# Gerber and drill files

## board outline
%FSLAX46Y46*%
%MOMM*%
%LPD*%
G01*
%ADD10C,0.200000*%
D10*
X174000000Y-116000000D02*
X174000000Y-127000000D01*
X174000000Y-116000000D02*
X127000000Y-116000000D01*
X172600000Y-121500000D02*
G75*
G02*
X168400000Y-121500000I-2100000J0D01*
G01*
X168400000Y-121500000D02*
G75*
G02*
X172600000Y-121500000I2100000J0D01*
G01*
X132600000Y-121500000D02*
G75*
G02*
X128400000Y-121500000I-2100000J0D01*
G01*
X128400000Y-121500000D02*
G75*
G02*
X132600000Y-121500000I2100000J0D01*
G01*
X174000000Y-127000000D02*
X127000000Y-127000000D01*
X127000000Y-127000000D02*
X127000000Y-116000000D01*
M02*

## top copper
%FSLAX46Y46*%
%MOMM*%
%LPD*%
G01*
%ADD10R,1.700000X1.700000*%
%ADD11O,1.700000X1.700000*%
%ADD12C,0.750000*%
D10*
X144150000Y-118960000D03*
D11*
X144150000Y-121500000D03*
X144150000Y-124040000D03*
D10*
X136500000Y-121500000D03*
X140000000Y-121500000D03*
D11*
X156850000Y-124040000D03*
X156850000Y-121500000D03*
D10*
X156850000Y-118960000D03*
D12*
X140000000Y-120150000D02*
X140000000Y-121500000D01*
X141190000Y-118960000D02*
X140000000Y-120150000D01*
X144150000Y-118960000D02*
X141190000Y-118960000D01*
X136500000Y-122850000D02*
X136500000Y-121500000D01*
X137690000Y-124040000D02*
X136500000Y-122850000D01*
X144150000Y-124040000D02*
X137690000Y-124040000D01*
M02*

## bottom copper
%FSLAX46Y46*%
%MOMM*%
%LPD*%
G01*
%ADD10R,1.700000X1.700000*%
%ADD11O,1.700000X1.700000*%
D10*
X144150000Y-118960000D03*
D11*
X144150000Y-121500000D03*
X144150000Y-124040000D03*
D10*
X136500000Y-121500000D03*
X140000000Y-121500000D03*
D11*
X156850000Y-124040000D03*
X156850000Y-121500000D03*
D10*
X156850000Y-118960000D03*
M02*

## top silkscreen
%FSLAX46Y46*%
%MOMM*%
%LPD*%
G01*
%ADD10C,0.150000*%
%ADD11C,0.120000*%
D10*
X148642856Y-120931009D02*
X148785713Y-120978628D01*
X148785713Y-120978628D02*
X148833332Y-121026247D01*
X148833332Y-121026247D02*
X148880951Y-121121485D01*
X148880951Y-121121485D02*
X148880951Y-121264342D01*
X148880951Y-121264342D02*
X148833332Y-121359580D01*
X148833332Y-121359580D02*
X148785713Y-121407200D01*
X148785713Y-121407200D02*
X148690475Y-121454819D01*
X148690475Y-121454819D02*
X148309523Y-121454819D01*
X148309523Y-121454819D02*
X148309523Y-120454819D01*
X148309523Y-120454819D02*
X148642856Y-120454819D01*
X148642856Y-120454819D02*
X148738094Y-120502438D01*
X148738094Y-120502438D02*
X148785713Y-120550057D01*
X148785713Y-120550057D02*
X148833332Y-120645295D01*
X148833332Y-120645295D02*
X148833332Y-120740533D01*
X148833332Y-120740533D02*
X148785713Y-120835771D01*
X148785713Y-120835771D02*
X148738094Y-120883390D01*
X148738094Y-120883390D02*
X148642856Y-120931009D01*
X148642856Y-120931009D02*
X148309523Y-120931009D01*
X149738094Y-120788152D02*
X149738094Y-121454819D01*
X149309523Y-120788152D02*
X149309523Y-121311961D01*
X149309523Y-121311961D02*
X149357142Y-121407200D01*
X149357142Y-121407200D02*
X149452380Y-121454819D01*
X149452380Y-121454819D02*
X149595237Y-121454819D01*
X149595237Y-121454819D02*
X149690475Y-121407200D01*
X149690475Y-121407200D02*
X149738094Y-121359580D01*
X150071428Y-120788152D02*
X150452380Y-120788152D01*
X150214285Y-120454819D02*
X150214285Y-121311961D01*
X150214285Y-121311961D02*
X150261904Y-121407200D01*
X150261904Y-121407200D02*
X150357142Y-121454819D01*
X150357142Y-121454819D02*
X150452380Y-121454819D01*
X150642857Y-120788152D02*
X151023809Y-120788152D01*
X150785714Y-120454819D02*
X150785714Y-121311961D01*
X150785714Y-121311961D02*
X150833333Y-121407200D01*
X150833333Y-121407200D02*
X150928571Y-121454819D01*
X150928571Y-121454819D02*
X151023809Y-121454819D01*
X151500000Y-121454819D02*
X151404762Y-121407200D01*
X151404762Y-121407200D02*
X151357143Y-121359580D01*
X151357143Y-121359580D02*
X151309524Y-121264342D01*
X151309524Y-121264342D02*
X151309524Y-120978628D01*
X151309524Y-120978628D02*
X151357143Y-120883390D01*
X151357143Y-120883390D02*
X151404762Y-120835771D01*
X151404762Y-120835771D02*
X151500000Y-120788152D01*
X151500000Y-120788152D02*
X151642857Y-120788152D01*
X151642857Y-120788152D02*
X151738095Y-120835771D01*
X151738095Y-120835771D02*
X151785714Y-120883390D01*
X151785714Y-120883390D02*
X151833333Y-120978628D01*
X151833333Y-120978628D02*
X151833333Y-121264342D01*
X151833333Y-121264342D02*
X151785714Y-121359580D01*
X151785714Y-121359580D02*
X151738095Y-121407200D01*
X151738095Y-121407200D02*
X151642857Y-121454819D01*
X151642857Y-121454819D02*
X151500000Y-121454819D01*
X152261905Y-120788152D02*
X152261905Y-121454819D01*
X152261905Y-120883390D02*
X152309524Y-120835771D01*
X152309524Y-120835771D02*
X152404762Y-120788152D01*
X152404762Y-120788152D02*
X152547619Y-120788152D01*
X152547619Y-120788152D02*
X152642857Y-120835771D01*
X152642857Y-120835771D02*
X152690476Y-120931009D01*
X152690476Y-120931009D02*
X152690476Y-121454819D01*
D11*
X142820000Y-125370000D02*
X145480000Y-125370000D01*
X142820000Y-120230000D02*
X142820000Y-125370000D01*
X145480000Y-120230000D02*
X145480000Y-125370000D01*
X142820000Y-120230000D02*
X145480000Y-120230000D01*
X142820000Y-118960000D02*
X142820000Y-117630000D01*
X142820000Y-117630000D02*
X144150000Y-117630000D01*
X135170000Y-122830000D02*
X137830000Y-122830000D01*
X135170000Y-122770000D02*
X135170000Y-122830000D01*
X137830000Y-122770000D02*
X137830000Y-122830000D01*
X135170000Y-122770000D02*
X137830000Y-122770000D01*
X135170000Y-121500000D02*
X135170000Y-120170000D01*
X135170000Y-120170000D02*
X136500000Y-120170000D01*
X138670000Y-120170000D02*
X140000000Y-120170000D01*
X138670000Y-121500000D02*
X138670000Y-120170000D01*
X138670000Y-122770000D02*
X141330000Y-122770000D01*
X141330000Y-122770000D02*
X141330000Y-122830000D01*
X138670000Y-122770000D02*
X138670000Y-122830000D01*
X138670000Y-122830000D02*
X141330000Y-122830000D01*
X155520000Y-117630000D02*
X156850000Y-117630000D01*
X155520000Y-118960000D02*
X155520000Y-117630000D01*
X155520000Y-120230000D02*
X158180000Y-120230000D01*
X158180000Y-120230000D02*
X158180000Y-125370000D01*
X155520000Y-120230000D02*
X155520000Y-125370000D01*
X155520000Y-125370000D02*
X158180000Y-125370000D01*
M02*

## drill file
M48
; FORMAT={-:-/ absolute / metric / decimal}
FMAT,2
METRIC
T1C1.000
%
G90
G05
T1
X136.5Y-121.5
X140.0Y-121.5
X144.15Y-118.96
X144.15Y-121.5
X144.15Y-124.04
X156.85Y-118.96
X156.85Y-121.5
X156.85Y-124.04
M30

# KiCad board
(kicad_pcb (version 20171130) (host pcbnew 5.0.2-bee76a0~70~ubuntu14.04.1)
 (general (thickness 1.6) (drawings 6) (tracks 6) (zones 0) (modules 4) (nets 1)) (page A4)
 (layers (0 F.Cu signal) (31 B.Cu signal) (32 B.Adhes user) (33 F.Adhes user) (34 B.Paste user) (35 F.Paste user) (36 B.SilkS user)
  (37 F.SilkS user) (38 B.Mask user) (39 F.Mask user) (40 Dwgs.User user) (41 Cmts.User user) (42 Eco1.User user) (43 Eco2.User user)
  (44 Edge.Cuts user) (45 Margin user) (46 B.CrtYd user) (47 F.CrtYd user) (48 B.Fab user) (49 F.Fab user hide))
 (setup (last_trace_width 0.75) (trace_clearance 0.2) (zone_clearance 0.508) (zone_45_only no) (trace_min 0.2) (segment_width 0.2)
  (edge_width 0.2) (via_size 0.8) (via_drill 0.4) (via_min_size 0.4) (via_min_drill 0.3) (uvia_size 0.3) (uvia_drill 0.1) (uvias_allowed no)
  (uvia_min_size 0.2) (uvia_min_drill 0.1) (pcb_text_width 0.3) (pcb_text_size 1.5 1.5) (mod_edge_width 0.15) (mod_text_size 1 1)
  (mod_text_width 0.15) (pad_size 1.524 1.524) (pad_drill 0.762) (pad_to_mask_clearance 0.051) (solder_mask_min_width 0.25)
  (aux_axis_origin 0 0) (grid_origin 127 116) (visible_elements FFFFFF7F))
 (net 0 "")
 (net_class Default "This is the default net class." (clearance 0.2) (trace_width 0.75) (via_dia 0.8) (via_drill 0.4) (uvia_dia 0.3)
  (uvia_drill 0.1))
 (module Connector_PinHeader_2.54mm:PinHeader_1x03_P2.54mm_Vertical (layer F.Cu) (at 144.15 118.96)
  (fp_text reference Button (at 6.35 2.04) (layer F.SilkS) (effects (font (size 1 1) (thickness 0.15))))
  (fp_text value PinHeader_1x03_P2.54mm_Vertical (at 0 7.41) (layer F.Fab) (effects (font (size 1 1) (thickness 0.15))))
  (fp_line (start -1.33 6.41) (end 1.33 6.41) (layer F.SilkS) (width 0.12))
  (fp_line (start -1.33 1.27) (end -1.33 6.41) (layer F.SilkS) (width 0.12))
  (fp_line (start 1.33 1.27) (end 1.33 6.41) (layer F.SilkS) (width 0.12))
  (fp_line (start -1.33 1.27) (end 1.33 1.27) (layer F.SilkS) (width 0.12))
  (fp_line (start -1.33 0) (end -1.33 -1.33) (layer F.SilkS) (width 0.12))
  (fp_line (start -1.33 -1.33) (end 0 -1.33) (layer F.SilkS) (width 0.12))
  (pad 1 thru_hole rect (at 0 0) (size 1.7 1.7) (drill 1) (layers *.Cu *.Mask))
  (pad 2 thru_hole oval (at 0 2.54) (size 1.7 1.7) (drill 1) (layers *.Cu *.Mask))
  (pad 3 thru_hole oval (at 0 5.08) (size 1.7 1.7) (drill 1) (layers *.Cu *.Mask)))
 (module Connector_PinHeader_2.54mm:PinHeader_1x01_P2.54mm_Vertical (layer F.Cu) (at 136.5 121.5)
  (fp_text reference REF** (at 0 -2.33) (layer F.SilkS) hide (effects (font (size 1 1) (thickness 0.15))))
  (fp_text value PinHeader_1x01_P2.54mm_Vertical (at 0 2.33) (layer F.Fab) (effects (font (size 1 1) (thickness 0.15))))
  (fp_line (start -1.33 1.33) (end 1.33 1.33) (layer F.SilkS) (width 0.12))
  (fp_line (start -1.33 1.27) (end -1.33 1.33) (layer F.SilkS) (width 0.12))
  (fp_line (start 1.33 1.27) (end 1.33 1.33) (layer F.SilkS) (width 0.12))
  (fp_line (start -1.33 1.27) (end 1.33 1.27) (layer F.SilkS) (width 0.12))
  (fp_line (start -1.33 0) (end -1.33 -1.33) (layer F.SilkS) (width 0.12))
  (fp_line (start -1.33 -1.33) (end 0 -1.33) (layer F.SilkS) (width 0.12))
  (pad 1 thru_hole rect (at 0 0) (size 1.7 1.7) (drill 1) (layers *.Cu *.Mask)))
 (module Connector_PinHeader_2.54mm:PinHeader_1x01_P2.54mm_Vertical (layer F.Cu) (at 140 121.5)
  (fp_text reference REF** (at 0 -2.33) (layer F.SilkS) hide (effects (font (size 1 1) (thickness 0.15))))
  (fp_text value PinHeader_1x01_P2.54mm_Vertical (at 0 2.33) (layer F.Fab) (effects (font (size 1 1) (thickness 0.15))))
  (fp_line (start -1.33 -1.33) (end 0 -1.33) (layer F.SilkS) (width 0.12))
  (fp_line (start -1.33 0) (end -1.33 -1.33) (layer F.SilkS) (width 0.12))
  (fp_line (start -1.33 1.27) (end 1.33 1.27) (layer F.SilkS) (width 0.12))
  (fp_line (start 1.33 1.27) (end 1.33 1.33) (layer F.SilkS) (width 0.12))
  (fp_line (start -1.33 1.27) (end -1.33 1.33) (layer F.SilkS) (width 0.12))
  (fp_line (start -1.33 1.33) (end 1.33 1.33) (layer F.SilkS) (width 0.12))
  (pad 1 thru_hole rect (at 0 0) (size 1.7 1.7) (drill 1) (layers *.Cu *.Mask)))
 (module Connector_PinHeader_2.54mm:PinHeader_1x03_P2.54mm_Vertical (layer F.Cu) (at 156.85 118.96)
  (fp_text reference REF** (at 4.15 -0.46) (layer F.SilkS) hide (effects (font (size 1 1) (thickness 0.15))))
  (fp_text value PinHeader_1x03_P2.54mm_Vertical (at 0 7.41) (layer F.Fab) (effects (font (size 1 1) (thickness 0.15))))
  (fp_line (start -1.33 -1.33) (end 0 -1.33) (layer F.SilkS) (width 0.12))
  (fp_line (start -1.33 0) (end -1.33 -1.33) (layer F.SilkS) (width 0.12))
  (fp_line (start -1.33 1.27) (end 1.33 1.27) (layer F.SilkS) (width 0.12))
  (fp_line (start 1.33 1.27) (end 1.33 6.41) (layer F.SilkS) (width 0.12))
  (fp_line (start -1.33 1.27) (end -1.33 6.41) (layer F.SilkS) (width 0.12))
  (fp_line (start -1.33 6.41) (end 1.33 6.41) (layer F.SilkS) (width 0.12))
  (pad 3 thru_hole oval (at 0 5.08) (size 1.7 1.7) (drill 1) (layers *.Cu *.Mask))
  (pad 2 thru_hole oval (at 0 2.54) (size 1.7 1.7) (drill 1) (layers *.Cu *.Mask))
  (pad 1 thru_hole rect (at 0 0) (size 1.7 1.7) (drill 1) (layers *.Cu *.Mask)))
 (gr_line (start 174 116) (end 174 127) (layer Edge.Cuts) (width 0.2))
 (gr_line (start 174 116) (end 127 116) (layer Edge.Cuts) (width 0.2))
 (gr_circle (center 170.5 121.5) (end 172.6 121.5) (layer Edge.Cuts) (width 0.2))
 (gr_circle (center 130.5 121.5) (end 132.6 121.5) (layer Edge.Cuts) (width 0.2))
 (gr_line (start 174 127) (end 127 127) (layer Edge.Cuts) (width 0.2))
 (gr_line (start 127 127) (end 127 116) (layer Edge.Cuts) (width 0.2))
 (segment (start 140 120.15) (end 140 121.5) (width 0.75) (layer F.Cu) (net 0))
 (segment (start 141.19 118.96) (end 140 120.15) (width 0.75) (layer F.Cu) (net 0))
 (segment (start 144.15 118.96) (end 141.19 118.96) (width 0.75) (layer F.Cu) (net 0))
 (segment (start 136.5 122.85) (end 136.5 121.5) (width 0.75) (layer F.Cu) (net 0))
 (segment (start 137.69 124.04) (end 136.5 122.85) (width 0.75) (layer F.Cu) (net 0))
 (segment (start 144.15 124.04) (end 137.69 124.04) (width 0.75) (layer F.Cu) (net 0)))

